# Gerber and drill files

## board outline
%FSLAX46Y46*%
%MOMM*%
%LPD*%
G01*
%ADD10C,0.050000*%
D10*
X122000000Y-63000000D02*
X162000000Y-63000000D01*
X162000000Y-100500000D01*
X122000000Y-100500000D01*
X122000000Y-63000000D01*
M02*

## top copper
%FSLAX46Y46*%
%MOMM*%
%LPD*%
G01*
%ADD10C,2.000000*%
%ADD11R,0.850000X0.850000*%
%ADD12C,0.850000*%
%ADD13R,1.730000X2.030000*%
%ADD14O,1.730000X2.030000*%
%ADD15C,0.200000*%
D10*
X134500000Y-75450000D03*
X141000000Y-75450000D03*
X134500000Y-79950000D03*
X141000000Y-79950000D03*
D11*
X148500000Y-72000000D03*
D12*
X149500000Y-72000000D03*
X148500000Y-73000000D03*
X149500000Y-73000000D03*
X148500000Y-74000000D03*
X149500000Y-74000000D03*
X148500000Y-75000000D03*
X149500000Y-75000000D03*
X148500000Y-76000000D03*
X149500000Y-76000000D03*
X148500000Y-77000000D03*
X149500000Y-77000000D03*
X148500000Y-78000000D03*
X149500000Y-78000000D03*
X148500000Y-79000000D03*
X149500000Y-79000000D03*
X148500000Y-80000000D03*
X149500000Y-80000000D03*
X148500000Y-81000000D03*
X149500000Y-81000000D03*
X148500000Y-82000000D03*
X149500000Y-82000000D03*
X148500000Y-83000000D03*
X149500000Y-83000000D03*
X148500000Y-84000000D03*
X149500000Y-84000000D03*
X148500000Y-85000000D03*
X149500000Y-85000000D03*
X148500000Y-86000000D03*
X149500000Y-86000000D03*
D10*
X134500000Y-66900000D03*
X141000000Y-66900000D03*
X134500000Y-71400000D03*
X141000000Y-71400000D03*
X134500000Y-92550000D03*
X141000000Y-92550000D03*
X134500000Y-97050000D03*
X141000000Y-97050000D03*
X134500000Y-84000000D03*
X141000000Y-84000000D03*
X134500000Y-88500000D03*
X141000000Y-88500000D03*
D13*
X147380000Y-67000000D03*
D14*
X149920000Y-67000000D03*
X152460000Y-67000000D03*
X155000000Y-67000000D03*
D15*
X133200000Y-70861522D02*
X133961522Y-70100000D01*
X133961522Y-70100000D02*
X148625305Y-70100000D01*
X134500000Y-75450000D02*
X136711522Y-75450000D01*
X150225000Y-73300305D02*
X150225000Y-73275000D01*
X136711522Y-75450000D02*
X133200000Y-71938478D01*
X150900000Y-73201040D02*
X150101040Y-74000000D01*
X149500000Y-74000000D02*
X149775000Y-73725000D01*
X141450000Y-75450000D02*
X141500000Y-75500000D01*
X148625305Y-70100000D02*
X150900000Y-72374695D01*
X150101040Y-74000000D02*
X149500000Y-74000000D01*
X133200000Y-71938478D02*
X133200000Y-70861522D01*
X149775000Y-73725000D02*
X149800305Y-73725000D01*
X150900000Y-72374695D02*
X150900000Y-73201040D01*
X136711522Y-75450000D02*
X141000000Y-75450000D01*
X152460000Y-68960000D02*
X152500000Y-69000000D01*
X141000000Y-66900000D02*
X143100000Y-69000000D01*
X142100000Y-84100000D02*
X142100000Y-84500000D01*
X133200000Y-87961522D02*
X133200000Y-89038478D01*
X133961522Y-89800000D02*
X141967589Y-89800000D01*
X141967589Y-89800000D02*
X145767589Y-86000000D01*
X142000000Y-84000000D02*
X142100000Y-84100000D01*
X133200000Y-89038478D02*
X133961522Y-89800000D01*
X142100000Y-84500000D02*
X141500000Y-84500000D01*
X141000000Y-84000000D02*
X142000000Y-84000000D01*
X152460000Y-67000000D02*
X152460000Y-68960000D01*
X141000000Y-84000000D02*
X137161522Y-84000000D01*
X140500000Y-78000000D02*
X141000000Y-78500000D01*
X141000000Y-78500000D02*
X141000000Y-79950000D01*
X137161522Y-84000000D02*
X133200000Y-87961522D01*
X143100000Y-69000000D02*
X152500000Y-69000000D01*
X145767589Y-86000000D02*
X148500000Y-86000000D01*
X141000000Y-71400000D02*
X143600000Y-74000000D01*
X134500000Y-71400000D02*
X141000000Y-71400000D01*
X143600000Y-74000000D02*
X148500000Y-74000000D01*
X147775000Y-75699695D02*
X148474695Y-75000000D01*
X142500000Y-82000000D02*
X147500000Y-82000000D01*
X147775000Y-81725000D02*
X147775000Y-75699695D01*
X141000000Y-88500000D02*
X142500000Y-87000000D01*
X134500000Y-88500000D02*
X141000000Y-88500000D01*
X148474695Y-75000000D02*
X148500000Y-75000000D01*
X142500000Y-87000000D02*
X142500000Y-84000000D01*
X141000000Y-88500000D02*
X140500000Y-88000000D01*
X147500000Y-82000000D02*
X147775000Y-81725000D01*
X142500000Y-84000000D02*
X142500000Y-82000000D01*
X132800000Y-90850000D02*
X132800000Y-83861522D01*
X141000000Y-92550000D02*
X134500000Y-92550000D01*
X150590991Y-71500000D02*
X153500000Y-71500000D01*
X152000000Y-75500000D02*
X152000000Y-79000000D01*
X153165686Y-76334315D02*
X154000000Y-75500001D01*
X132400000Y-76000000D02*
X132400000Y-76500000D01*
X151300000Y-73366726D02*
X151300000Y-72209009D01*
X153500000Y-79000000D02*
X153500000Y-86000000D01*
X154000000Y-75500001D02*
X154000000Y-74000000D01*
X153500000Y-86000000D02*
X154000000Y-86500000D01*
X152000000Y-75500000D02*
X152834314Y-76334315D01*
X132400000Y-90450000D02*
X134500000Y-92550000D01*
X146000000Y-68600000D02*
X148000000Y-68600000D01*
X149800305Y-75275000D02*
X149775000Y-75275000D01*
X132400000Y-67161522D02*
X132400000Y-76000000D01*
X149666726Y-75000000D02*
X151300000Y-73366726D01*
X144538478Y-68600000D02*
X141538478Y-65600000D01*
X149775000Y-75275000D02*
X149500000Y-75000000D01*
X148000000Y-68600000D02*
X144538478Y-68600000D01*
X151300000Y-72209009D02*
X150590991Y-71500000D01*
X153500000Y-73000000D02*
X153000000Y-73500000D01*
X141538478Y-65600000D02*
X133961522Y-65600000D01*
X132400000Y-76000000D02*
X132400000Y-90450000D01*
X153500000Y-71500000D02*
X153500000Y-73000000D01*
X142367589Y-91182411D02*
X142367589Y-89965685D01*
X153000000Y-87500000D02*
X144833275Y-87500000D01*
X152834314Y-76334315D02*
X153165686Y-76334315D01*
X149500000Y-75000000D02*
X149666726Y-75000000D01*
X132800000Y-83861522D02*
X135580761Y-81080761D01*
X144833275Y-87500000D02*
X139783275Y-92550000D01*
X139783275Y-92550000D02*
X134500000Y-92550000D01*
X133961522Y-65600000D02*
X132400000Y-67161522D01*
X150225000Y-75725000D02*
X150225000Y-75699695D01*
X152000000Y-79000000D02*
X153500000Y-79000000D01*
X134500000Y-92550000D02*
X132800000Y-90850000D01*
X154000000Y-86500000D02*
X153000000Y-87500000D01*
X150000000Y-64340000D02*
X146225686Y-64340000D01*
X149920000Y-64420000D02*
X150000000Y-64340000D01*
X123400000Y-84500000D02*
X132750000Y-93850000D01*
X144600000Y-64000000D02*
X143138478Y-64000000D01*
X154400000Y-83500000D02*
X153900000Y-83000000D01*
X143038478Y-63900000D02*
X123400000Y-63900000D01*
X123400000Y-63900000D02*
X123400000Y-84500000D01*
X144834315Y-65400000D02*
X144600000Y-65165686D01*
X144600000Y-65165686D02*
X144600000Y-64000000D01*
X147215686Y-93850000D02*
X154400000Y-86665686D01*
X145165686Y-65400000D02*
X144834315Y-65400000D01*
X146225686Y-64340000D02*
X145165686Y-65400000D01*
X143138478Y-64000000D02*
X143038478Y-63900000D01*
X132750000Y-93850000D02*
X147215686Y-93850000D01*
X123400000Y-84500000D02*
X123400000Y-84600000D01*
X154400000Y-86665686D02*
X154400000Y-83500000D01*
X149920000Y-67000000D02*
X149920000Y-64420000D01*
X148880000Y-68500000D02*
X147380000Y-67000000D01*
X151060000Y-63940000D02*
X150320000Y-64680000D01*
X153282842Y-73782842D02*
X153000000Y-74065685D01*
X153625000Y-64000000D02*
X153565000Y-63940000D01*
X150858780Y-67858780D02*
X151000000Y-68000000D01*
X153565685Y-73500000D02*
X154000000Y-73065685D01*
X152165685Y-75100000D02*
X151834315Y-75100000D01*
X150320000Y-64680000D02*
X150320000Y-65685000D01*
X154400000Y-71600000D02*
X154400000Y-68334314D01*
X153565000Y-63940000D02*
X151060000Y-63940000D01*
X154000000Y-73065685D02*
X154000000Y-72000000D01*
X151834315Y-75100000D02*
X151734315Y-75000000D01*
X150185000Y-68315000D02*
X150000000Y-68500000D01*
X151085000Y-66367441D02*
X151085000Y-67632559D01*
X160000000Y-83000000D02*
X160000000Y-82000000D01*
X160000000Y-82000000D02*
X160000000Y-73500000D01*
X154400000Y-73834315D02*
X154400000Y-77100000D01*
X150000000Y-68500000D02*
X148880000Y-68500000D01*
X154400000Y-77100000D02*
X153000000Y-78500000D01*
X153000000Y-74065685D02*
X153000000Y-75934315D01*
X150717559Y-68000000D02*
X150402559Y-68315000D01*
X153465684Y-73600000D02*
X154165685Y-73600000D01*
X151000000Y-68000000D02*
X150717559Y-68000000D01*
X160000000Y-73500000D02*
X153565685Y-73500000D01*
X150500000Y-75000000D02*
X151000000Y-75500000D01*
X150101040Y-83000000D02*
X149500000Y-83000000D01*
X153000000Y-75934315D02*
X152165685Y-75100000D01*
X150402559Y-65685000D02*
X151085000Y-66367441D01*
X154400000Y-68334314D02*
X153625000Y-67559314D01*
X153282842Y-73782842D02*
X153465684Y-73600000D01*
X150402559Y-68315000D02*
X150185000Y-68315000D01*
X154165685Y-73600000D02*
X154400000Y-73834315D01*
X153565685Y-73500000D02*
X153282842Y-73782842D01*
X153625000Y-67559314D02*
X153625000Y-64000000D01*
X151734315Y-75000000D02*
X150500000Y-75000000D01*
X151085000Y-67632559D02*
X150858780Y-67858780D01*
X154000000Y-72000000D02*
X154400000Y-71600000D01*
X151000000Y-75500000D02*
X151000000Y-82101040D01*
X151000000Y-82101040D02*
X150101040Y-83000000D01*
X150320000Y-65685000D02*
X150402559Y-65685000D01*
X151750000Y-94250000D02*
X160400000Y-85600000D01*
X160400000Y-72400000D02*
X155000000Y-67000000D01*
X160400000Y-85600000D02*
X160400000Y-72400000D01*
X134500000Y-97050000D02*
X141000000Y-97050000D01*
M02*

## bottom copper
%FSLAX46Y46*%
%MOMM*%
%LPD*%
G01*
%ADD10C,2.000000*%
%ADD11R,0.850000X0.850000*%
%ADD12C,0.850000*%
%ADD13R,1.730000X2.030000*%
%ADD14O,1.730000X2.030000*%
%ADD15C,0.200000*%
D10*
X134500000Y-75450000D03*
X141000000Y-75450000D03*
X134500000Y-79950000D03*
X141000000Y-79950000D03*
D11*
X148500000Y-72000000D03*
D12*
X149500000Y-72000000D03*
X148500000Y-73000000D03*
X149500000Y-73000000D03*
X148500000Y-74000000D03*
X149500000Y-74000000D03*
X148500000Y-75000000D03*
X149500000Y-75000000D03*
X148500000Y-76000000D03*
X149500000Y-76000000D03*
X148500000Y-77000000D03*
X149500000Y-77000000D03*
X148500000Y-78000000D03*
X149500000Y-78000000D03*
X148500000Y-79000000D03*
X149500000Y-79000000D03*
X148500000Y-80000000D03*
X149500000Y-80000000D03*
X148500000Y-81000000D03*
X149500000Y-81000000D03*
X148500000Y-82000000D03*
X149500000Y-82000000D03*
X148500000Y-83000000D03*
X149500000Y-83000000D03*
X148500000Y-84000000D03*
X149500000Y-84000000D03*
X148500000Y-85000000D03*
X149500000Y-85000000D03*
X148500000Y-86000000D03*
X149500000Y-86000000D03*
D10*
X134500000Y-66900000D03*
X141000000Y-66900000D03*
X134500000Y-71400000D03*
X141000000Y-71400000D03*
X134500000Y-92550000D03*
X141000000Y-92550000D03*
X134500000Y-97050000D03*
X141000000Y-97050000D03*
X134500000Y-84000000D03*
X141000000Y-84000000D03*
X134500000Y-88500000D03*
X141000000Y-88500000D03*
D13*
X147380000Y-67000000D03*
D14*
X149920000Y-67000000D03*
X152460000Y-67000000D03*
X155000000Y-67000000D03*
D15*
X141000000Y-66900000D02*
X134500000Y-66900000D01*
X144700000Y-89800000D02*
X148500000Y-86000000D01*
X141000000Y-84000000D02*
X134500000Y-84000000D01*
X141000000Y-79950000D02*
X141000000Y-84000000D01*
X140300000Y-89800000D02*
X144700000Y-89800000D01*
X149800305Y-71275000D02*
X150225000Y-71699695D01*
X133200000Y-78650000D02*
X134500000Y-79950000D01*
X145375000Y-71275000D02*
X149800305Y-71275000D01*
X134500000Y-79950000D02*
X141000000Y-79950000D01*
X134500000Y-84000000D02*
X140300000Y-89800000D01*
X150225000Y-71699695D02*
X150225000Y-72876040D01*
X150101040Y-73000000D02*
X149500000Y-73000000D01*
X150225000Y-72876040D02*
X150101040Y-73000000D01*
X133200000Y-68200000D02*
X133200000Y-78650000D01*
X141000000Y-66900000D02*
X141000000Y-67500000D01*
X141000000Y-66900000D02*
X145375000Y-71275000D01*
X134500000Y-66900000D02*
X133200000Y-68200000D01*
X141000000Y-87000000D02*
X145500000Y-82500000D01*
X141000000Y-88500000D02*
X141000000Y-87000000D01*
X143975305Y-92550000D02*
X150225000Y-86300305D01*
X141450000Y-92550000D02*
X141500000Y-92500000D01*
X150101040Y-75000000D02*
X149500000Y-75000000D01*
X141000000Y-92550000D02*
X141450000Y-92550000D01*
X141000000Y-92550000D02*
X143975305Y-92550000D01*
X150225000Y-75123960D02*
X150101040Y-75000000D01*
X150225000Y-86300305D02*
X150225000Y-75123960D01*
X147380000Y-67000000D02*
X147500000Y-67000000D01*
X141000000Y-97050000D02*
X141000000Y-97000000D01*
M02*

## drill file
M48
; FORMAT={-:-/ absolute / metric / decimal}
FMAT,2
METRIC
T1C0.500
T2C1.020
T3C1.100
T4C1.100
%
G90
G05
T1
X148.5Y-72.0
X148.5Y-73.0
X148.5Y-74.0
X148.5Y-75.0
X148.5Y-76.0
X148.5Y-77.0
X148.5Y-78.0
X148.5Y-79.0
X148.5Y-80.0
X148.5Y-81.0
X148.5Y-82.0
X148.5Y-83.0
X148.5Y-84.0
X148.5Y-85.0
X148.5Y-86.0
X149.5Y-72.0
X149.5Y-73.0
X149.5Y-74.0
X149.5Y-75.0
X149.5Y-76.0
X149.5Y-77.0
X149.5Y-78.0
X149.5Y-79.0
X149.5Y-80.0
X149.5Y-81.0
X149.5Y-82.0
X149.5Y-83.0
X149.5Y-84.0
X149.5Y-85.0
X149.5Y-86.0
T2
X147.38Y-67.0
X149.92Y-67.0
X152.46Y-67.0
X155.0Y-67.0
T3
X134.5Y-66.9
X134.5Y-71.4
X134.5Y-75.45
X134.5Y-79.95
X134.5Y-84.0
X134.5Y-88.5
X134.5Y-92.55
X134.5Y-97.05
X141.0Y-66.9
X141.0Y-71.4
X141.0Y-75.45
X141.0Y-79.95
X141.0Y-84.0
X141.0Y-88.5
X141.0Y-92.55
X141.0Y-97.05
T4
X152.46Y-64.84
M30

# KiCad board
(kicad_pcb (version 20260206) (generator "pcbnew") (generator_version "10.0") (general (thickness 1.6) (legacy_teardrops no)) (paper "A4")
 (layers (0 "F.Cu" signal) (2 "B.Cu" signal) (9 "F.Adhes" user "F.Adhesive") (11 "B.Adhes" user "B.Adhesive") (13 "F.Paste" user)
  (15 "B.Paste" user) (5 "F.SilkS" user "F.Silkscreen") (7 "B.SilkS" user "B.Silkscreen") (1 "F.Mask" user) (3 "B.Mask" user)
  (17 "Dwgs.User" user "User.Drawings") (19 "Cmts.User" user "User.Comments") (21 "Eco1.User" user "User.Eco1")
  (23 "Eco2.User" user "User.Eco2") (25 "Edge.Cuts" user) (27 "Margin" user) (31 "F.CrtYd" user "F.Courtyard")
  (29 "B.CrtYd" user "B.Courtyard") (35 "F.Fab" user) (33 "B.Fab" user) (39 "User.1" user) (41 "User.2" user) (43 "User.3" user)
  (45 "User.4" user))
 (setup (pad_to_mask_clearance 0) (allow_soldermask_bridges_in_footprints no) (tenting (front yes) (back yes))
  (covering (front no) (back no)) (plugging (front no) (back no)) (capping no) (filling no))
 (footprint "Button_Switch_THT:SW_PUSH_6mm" (layer "F.Cu") (at 134.5 75.45)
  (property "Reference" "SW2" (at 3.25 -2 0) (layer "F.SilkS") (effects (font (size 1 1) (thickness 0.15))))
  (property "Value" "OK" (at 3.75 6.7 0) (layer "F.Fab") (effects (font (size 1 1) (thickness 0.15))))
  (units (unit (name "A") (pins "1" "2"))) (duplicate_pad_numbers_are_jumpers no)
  (pad "1" thru_hole circle (at 0 0 90) (size 2 2) (drill 1.1) (layers "*.Cu" "*.Mask") (remove_unused_layers no) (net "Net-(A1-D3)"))
  (pad "1" thru_hole circle (at 6.5 0 90) (size 2 2) (drill 1.1) (layers "*.Cu" "*.Mask") (remove_unused_layers no) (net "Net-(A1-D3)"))
  (pad "2" thru_hole circle (at 0 4.5 90) (size 2 2) (drill 1.1) (layers "*.Cu" "*.Mask") (remove_unused_layers no) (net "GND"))
  (pad "2" thru_hole circle (at 6.5 4.5 90) (size 2 2) (drill 1.1) (layers "*.Cu" "*.Mask") (remove_unused_layers no) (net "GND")))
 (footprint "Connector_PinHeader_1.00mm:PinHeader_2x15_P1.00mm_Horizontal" (layer "F.Cu") (at 148.5 72)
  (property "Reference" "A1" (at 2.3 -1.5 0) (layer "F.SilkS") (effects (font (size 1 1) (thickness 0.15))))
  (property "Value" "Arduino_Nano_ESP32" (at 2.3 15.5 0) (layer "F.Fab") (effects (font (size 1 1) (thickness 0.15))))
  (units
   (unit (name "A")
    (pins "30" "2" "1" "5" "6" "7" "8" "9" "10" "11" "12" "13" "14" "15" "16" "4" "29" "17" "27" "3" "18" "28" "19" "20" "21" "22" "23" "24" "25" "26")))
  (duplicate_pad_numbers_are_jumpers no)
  (pad "1" thru_hole rect (at 0 0) (size 0.85 0.85) (drill 0.5) (layers "*.Cu" "*.Mask") (remove_unused_layers no)
   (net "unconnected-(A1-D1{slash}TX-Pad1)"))
  (pad "2" thru_hole circle (at 1 0) (size 0.85 0.85) (drill 0.5) (layers "*.Cu" "*.Mask") (remove_unused_layers no)
   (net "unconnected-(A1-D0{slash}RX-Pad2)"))
  (pad "3" thru_hole circle (at 0 1) (size 0.85 0.85) (drill 0.5) (layers "*.Cu" "*.Mask") (remove_unused_layers no)
   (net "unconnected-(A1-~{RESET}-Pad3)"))
  (pad "4" thru_hole circle (at 1 1) (size 0.85 0.85) (drill 0.5) (layers "*.Cu" "*.Mask") (remove_unused_layers no) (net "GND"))
  (pad "5" thru_hole circle (at 0 2) (size 0.85 0.85) (drill 0.5) (layers "*.Cu" "*.Mask") (remove_unused_layers no) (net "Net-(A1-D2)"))
  (pad "6" thru_hole circle (at 1 2) (size 0.85 0.85) (drill 0.5) (layers "*.Cu" "*.Mask") (remove_unused_layers no) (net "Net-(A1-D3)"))
  (pad "7" thru_hole circle (at 0 3) (size 0.85 0.85) (drill 0.5) (layers "*.Cu" "*.Mask") (remove_unused_layers no) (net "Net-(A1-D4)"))
  (pad "8" thru_hole circle (at 1 3) (size 0.85 0.85) (drill 0.5) (layers "*.Cu" "*.Mask") (remove_unused_layers no) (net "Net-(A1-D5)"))
  (pad "9" thru_hole circle (at 0 4) (size 0.85 0.85) (drill 0.5) (layers "*.Cu" "*.Mask") (remove_unused_layers no)
   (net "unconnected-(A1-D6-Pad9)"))
  (pad "10" thru_hole circle (at 1 4) (size 0.85 0.85) (drill 0.5) (layers "*.Cu" "*.Mask") (remove_unused_layers no)
   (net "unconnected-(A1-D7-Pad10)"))
  (pad "11" thru_hole circle (at 0 5) (size 0.85 0.85) (drill 0.5) (layers "*.Cu" "*.Mask") (remove_unused_layers no)
   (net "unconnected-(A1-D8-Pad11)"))
  (pad "12" thru_hole circle (at 1 5) (size 0.85 0.85) (drill 0.5) (layers "*.Cu" "*.Mask") (remove_unused_layers no)
   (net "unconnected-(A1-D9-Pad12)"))
  (pad "13" thru_hole circle (at 0 6) (size 0.85 0.85) (drill 0.5) (layers "*.Cu" "*.Mask") (remove_unused_layers no)
   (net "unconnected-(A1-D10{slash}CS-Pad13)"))
  (pad "14" thru_hole circle (at 1 6) (size 0.85 0.85) (drill 0.5) (layers "*.Cu" "*.Mask") (remove_unused_layers no)
   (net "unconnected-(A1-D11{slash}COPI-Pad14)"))
  (pad "15" thru_hole circle (at 0 7) (size 0.85 0.85) (drill 0.5) (layers "*.Cu" "*.Mask") (remove_unused_layers no)
   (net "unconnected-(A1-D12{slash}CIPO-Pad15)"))
  (pad "16" thru_hole circle (at 1 7) (size 0.85 0.85) (drill 0.5) (layers "*.Cu" "*.Mask") (remove_unused_layers no)
   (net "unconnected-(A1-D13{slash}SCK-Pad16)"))
  (pad "17" thru_hole circle (at 0 8) (size 0.85 0.85) (drill 0.5) (layers "*.Cu" "*.Mask") (remove_unused_layers no)
   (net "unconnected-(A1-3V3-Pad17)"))
  (pad "18" thru_hole circle (at 1 8) (size 0.85 0.85) (drill 0.5) (layers "*.Cu" "*.Mask") (remove_unused_layers no)
   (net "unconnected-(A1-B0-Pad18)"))
  (pad "19" thru_hole circle (at 0 9) (size 0.85 0.85) (drill 0.5) (layers "*.Cu" "*.Mask") (remove_unused_layers no)
   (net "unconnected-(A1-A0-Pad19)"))
  (pad "20" thru_hole circle (at 1 9) (size 0.85 0.85) (drill 0.5) (layers "*.Cu" "*.Mask") (remove_unused_layers no)
   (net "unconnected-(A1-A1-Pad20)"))
  (pad "21" thru_hole circle (at 0 10) (size 0.85 0.85) (drill 0.5) (layers "*.Cu" "*.Mask") (remove_unused_layers no)
   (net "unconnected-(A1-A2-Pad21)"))
  (pad "22" thru_hole circle (at 1 10) (size 0.85 0.85) (drill 0.5) (layers "*.Cu" "*.Mask") (remove_unused_layers no)
   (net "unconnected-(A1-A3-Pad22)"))
  (pad "23" thru_hole circle (at 0 11) (size 0.85 0.85) (drill 0.5) (layers "*.Cu" "*.Mask") (remove_unused_layers no)
   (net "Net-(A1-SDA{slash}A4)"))
  (pad "24" thru_hole circle (at 1 11) (size 0.85 0.85) (drill 0.5) (layers "*.Cu" "*.Mask") (remove_unused_layers no)
   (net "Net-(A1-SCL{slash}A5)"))
  (pad "25" thru_hole circle (at 0 12) (size 0.85 0.85) (drill 0.5) (layers "*.Cu" "*.Mask") (remove_unused_layers no)
   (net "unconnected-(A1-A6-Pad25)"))
  (pad "26" thru_hole circle (at 1 12) (size 0.85 0.85) (drill 0.5) (layers "*.Cu" "*.Mask") (remove_unused_layers no)
   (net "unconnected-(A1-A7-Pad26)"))
  (pad "27" thru_hole circle (at 0 13) (size 0.85 0.85) (drill 0.5) (layers "*.Cu" "*.Mask") (remove_unused_layers no)
   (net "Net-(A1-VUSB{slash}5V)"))
  (pad "28" thru_hole circle (at 1 13) (size 0.85 0.85) (drill 0.5) (layers "*.Cu" "*.Mask") (remove_unused_layers no)
   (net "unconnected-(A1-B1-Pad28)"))
  (pad "29" thru_hole circle (at 0 14) (size 0.85 0.85) (drill 0.5) (layers "*.Cu" "*.Mask") (remove_unused_layers no) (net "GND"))
  (pad "30" thru_hole circle (at 1 14) (size 0.85 0.85) (drill 0.5) (layers "*.Cu" "*.Mask") (remove_unused_layers no)
   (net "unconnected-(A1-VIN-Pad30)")))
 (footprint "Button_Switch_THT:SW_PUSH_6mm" (layer "F.Cu") (at 134.5 66.9)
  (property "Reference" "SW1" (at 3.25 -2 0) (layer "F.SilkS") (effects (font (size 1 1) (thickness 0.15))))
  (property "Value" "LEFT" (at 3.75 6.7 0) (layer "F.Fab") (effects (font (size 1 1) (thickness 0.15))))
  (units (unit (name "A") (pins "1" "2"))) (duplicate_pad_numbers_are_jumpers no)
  (pad "1" thru_hole circle (at 0 0 90) (size 2 2) (drill 1.1) (layers "*.Cu" "*.Mask") (remove_unused_layers no) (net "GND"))
  (pad "1" thru_hole circle (at 6.5 0 90) (size 2 2) (drill 1.1) (layers "*.Cu" "*.Mask") (remove_unused_layers no) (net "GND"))
  (pad "2" thru_hole circle (at 0 4.5 90) (size 2 2) (drill 1.1) (layers "*.Cu" "*.Mask") (remove_unused_layers no) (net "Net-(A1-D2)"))
  (pad "2" thru_hole circle (at 6.5 4.5 90) (size 2 2) (drill 1.1) (layers "*.Cu" "*.Mask") (remove_unused_layers no) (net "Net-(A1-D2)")))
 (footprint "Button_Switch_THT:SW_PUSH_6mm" (layer "F.Cu") (at 134.5 92.55)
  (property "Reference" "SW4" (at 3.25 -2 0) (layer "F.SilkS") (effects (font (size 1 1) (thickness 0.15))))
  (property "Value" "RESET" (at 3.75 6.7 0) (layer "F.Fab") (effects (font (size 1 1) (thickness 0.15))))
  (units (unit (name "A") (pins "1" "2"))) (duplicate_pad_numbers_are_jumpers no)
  (pad "1" thru_hole circle (at 0 0 90) (size 2 2) (drill 1.1) (layers "*.Cu" "*.Mask") (remove_unused_layers no) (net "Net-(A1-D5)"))
  (pad "1" thru_hole circle (at 6.5 0 90) (size 2 2) (drill 1.1) (layers "*.Cu" "*.Mask") (remove_unused_layers no) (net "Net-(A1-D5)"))
  (pad "2" thru_hole circle (at 0 4.5 90) (size 2 2) (drill 1.1) (layers "*.Cu" "*.Mask") (remove_unused_layers no)
   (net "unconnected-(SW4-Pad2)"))
  (pad "2" thru_hole circle (at 6.5 4.5 90) (size 2 2) (drill 1.1) (layers "*.Cu" "*.Mask") (remove_unused_layers no)
   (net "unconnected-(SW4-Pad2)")))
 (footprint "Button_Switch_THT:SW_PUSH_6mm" (layer "F.Cu") (at 134.5 84)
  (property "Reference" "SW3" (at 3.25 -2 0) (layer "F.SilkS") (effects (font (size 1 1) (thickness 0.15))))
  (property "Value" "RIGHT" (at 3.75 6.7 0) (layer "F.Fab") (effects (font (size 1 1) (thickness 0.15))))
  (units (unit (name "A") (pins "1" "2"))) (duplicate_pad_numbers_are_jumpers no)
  (pad "1" thru_hole circle (at 0 0 90) (size 2 2) (drill 1.1) (layers "*.Cu" "*.Mask") (remove_unused_layers no) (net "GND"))
  (pad "1" thru_hole circle (at 6.5 0 90) (size 2 2) (drill 1.1) (layers "*.Cu" "*.Mask") (remove_unused_layers no) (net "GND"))
  (pad "2" thru_hole circle (at 0 4.5 90) (size 2 2) (drill 1.1) (layers "*.Cu" "*.Mask") (remove_unused_layers no) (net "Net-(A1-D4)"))
  (pad "2" thru_hole circle (at 6.5 4.5 90) (size 2 2) (drill 1.1) (layers "*.Cu" "*.Mask") (remove_unused_layers no) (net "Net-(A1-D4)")))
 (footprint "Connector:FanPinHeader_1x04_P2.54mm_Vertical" (layer "F.Cu") (at 147.38 67)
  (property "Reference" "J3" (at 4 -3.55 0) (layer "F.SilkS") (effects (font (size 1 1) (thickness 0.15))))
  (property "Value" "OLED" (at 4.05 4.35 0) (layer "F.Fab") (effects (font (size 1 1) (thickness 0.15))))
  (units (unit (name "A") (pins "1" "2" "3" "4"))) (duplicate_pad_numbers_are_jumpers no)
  (pad "" np_thru_hole circle (at 5.08 -2.16 90) (size 1.1 1.1) (drill 1.1) (layers "*.Cu" "*.Mask"))
  (pad "1" thru_hole rect (at 0 0 90) (size 2.03 1.73) (drill 1.02) (layers "*.Cu" "*.Mask") (remove_unused_layers no)
   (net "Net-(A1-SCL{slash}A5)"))
  (pad "2" thru_hole oval (at 2.54 0 90) (size 2.03 1.73) (drill 1.02) (layers "*.Cu" "*.Mask") (remove_unused_layers no)
   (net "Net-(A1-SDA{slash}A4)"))
  (pad "3" thru_hole oval (at 5.08 0 90) (size 2.03 1.73) (drill 1.02) (layers "*.Cu" "*.Mask") (remove_unused_layers no) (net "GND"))
  (pad "4" thru_hole oval (at 7.62 0 90) (size 2.03 1.73) (drill 1.02) (layers "*.Cu" "*.Mask") (remove_unused_layers no)
   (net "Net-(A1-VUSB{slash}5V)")))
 (gr_rect (start 122 63) (end 162 100.5) (stroke (width 0.05) (type default)) (fill no) (layer "Edge.Cuts"))
 (segment (start 133.2 70.861522) (end 133.961522 70.1) (width 0.2) (layer "F.Cu") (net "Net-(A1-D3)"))
 (segment (start 133.961522 70.1) (end 148.625305 70.1) (width 0.2) (layer "F.Cu") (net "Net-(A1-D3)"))
 (segment (start 134.5 75.45) (end 136.711522 75.45) (width 0.2) (layer "F.Cu") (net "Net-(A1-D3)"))
 (segment (start 150.225 73.300305) (end 150.225 73.275) (width 0.2) (layer "F.Cu") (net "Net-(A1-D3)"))
 (segment (start 136.711522 75.45) (end 133.2 71.938478) (width 0.2) (layer "F.Cu") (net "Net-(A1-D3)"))
 (segment (start 150.9 73.20104) (end 150.10104 74) (width 0.2) (layer "F.Cu") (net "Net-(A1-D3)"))
 (segment (start 149.5 74) (end 149.775 73.725) (width 0.2) (layer "F.Cu") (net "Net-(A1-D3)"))
 (segment (start 141.45 75.45) (end 141.5 75.5) (width 0.2) (layer "F.Cu") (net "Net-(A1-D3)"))
 (segment (start 148.625305 70.1) (end 150.9 72.374695) (width 0.2) (layer "F.Cu") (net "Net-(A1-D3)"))
 (segment (start 150.10104 74) (end 149.5 74) (width 0.2) (layer "F.Cu") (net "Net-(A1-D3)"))
 (segment (start 133.2 71.938478) (end 133.2 70.861522) (width 0.2) (layer "F.Cu") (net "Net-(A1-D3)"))
 (segment (start 149.775 73.725) (end 149.800305 73.725) (width 0.2) (layer "F.Cu") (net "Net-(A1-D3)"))
 (segment (start 150.9 72.374695) (end 150.9 73.20104) (width 0.2) (layer "F.Cu") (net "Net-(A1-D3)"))
 (segment (start 136.711522 75.45) (end 141 75.45) (width 0.2) (layer "F.Cu") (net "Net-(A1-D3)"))
 (segment (start 152.46 68.96) (end 152.5 69) (width 0.2) (layer "F.Cu") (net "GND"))
 (segment (start 141 66.9) (end 143.1 69) (width 0.2) (layer "F.Cu") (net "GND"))
 (segment (start 142.1 84.1) (end 142.1 84.5) (width 0.2) (layer "F.Cu") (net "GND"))
 (segment (start 133.2 87.961522) (end 133.2 89.038478) (width 0.2) (layer "F.Cu") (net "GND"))
 (segment (start 133.961522 89.8) (end 141.967589 89.8) (width 0.2) (layer "F.Cu") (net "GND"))
 (segment (start 141.967589 89.8) (end 145.767589 86) (width 0.2) (layer "F.Cu") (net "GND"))
 (segment (start 142 84) (end 142.1 84.1) (width 0.2) (layer "F.Cu") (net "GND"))
 (segment (start 133.2 89.038478) (end 133.961522 89.8) (width 0.2) (layer "F.Cu") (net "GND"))
 (segment (start 142.1 84.5) (end 141.5 84.5) (width 0.2) (layer "F.Cu") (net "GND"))
 (segment (start 141 84) (end 142 84) (width 0.2) (layer "F.Cu") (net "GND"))
 (segment (start 152.46 67) (end 152.46 68.96) (width 0.2) (layer "F.Cu") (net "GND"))
 (segment (start 141 84) (end 137.161522 84) (width 0.2) (layer "F.Cu") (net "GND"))
 (segment (start 140.5 78) (end 141 78.5) (width 0.2) (layer "F.Cu") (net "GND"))
 (segment (start 141 78.5) (end 141 79.95) (width 0.2) (layer "F.Cu") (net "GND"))
 (segment (start 137.161522 84) (end 133.2 87.961522) (width 0.2) (layer "F.Cu") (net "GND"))
 (segment (start 143.1 69) (end 152.5 69) (width 0.2) (layer "F.Cu") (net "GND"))
 (segment (start 145.767589 86) (end 148.5 86) (width 0.2) (layer "F.Cu") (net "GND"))
 (segment (start 141 66.9) (end 134.5 66.9) (width 0.2) (layer "B.Cu") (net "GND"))
 (segment (start 144.7 89.8) (end 148.5 86) (width 0.2) (layer "B.Cu") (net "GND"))
 (segment (start 141 84) (end 134.5 84) (width 0.2) (layer "B.Cu") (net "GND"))
 (segment (start 141 79.95) (end 141 84) (width 0.2) (layer "B.Cu") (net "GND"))
 (segment (start 140.3 89.8) (end 144.7 89.8) (width 0.2) (layer "B.Cu") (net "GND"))
 (segment (start 149.800305 71.275) (end 150.225 71.699695) (width 0.2) (layer "B.Cu") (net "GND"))
 (segment (start 133.2 78.65) (end 134.5 79.95) (width 0.2) (layer "B.Cu") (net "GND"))
 (segment (start 145.375 71.275) (end 149.800305 71.275) (width 0.2) (layer "B.Cu") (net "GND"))
 (segment (start 134.5 79.95) (end 141 79.95) (width 0.2) (layer "B.Cu") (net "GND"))
 (segment (start 134.5 84) (end 140.3 89.8) (width 0.2) (layer "B.Cu") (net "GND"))
 (segment (start 150.225 71.699695) (end 150.225 72.87604) (width 0.2) (layer "B.Cu") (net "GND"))
 (segment (start 150.10104 73) (end 149.5 73) (width 0.2) (layer "B.Cu") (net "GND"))
 (segment (start 150.225 72.87604) (end 150.10104 73) (width 0.2) (layer "B.Cu") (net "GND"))
 (segment (start 133.2 68.2) (end 133.2 78.65) (width 0.2) (layer "B.Cu") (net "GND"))
 (segment (start 141 66.9) (end 141 67.5) (width 0.2) (layer "B.Cu") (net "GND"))
 (segment (start 141 66.9) (end 145.375 71.275) (width 0.2) (layer "B.Cu") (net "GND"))
 (segment (start 134.5 66.9) (end 133.2 68.2) (width 0.2) (layer "B.Cu") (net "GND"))
 (segment (start 141 71.4) (end 143.6 74) (width 0.2) (layer "F.Cu") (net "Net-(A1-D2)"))
 (segment (start 134.5 71.4) (end 141 71.4) (width 0.2) (layer "F.Cu") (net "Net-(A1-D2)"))
 (segment (start 143.6 74) (end 148.5 74) (width 0.2) (layer "F.Cu") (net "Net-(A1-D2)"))
 (segment (start 147.775 75.699695) (end 148.474695 75) (width 0.2) (layer "F.Cu") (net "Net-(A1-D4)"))
 (segment (start 142.5 82) (end 147.5 82) (width 0.2) (layer "F.Cu") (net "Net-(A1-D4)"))
 (segment (start 147.775 81.725) (end 147.775 75.699695) (width 0.2) (layer "F.Cu") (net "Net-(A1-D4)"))
 (segment (start 141 88.5) (end 142.5 87) (width 0.2) (layer "F.Cu") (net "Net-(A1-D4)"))
 (segment (start 134.5 88.5) (end 141 88.5) (width 0.2) (layer "F.Cu") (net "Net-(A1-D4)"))
 (segment (start 148.474695 75) (end 148.5 75) (width 0.2) (layer "F.Cu") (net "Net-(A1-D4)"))
 (segment (start 142.5 87) (end 142.5 84) (width 0.2) (layer "F.Cu") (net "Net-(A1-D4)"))
 (segment (start 141 88.5) (end 140.5 88) (width 0.2) (layer "F.Cu") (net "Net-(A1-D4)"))
 (segment (start 147.5 82) (end 147.775 81.725) (width 0.2) (layer "F.Cu") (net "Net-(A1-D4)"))
 (segment (start 142.5 84) (end 142.5 82) (width 0.2) (layer "F.Cu") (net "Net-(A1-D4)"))
 (segment (start 141 87) (end 145.5 82.5) (width 0.2) (layer "B.Cu") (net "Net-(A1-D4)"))
 (segment (start 141 88.5) (end 141 87) (width 0.2) (layer "B.Cu") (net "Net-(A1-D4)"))
 (segment (start 132.8 90.85) (end 132.8 83.861522) (width 0.2) (layer "F.Cu") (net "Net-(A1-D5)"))
 (segment (start 141 92.55) (end 134.5 92.55) (width 0.2) (layer "F.Cu") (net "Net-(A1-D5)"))
 (segment (start 150.590991 71.5) (end 153.5 71.5) (width 0.2) (layer "F.Cu") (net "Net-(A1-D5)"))
 (segment (start 152 75.5) (end 152 79) (width 0.2) (layer "F.Cu") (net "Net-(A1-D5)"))
 (segment (start 153.165686 76.334315) (end 154 75.500001) (width 0.2) (layer "F.Cu") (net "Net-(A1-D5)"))
 (segment (start 132.4 76) (end 132.4 76.5) (width 0.2) (layer "F.Cu") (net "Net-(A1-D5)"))
 (segment (start 151.3 73.366726) (end 151.3 72.209009) (width 0.2) (layer "F.Cu") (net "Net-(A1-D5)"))
 (segment (start 153.5 79) (end 153.5 86) (width 0.2) (layer "F.Cu") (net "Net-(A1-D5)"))
 (segment (start 154 75.500001) (end 154 74) (width 0.2) (layer "F.Cu") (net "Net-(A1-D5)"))
 (segment (start 153.5 86) (end 154 86.5) (width 0.2) (layer "F.Cu") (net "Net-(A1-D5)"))
 (segment (start 152 75.5) (end 152.834314 76.334315) (width 0.2) (layer "F.Cu") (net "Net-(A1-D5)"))
 (segment (start 132.4 90.45) (end 134.5 92.55) (width 0.2) (layer "F.Cu") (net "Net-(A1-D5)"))
 (segment (start 146 68.6) (end 148 68.6) (width 0.2) (layer "F.Cu") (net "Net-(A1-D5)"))
 (segment (start 149.800305 75.275) (end 149.775 75.275) (width 0.2) (layer "F.Cu") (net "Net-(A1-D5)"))
 (segment (start 132.4 67.161522) (end 132.4 76) (width 0.2) (layer "F.Cu") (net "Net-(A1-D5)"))
 (segment (start 149.666726 75) (end 151.3 73.366726) (width 0.2) (layer "F.Cu") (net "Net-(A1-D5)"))
 (segment (start 144.538478 68.6) (end 141.538478 65.6) (width 0.2) (layer "F.Cu") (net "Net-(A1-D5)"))
 (segment (start 149.775 75.275) (end 149.5 75) (width 0.2) (layer "F.Cu") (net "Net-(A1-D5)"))
 (segment (start 148 68.6) (end 144.538478 68.6) (width 0.2) (layer "F.Cu") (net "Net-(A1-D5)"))
 (segment (start 151.3 72.209009) (end 150.590991 71.5) (width 0.2) (layer "F.Cu") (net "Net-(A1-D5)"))
 (segment (start 153.5 73) (end 153 73.5) (width 0.2) (layer "F.Cu") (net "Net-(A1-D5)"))
 (segment (start 141.538478 65.6) (end 133.961522 65.6) (width 0.2) (layer "F.Cu") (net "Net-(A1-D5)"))
 (segment (start 132.4 76) (end 132.4 90.45) (width 0.2) (layer "F.Cu") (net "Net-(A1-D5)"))
 (segment (start 153.5 71.5) (end 153.5 73) (width 0.2) (layer "F.Cu") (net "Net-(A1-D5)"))
 (segment (start 142.367589 91.182411) (end 142.367589 89.965685) (width 0.2) (layer "F.Cu") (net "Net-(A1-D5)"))
 (segment (start 153 87.5) (end 144.833275 87.5) (width 0.2) (layer "F.Cu") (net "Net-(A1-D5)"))
 (segment (start 152.834314 76.334315) (end 153.165686 76.334315) (width 0.2) (layer "F.Cu") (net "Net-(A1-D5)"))
 (segment (start 149.5 75) (end 149.666726 75) (width 0.2) (layer "F.Cu") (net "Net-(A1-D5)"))
 (segment (start 132.8 83.861522) (end 135.580761 81.080761) (width 0.2) (layer "F.Cu") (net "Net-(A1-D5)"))
 (segment (start 144.833275 87.5) (end 139.783275 92.55) (width 0.2) (layer "F.Cu") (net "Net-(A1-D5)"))
 (segment (start 139.783275 92.55) (end 134.5 92.55) (width 0.2) (layer "F.Cu") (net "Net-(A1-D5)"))
 (segment (start 133.961522 65.6) (end 132.4 67.161522) (width 0.2) (layer "F.Cu") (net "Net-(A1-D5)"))
 (segment (start 150.225 75.725) (end 150.225 75.699695) (width 0.2) (layer "F.Cu") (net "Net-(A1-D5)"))
 (segment (start 152 79) (end 153.5 79) (width 0.2) (layer "F.Cu") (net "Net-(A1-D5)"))
 (segment (start 134.5 92.55) (end 132.8 90.85) (width 0.2) (layer "F.Cu") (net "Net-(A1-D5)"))
 (segment (start 154 86.5) (end 153 87.5) (width 0.2) (layer "F.Cu") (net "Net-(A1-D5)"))
 (segment (start 143.975305 92.55) (end 150.225 86.300305) (width 0.2) (layer "B.Cu") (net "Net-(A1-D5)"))
 (segment (start 141.45 92.55) (end 141.5 92.5) (width 0.2) (layer "B.Cu") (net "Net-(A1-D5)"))
 (segment (start 150.10104 75) (end 149.5 75) (width 0.2) (layer "B.Cu") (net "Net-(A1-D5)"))
 (segment (start 141 92.55) (end 141.45 92.55) (width 0.2) (layer "B.Cu") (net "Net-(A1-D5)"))
 (segment (start 141 92.55) (end 143.975305 92.55) (width 0.2) (layer "B.Cu") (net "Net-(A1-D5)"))
 (segment (start 150.225 75.12396) (end 150.10104 75) (width 0.2) (layer "B.Cu") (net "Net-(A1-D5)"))
 (segment (start 150.225 86.300305) (end 150.225 75.12396) (width 0.2) (layer "B.Cu") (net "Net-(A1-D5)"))
 (segment (start 150 64.34) (end 146.225686 64.34) (width 0.2) (layer "F.Cu") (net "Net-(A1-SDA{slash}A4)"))
 (segment (start 149.92 64.42) (end 150 64.34) (width 0.2) (layer "F.Cu") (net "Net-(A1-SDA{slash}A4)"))
 (segment (start 123.4 84.5) (end 132.75 93.85) (width 0.2) (layer "F.Cu") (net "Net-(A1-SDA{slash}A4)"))
 (segment (start 144.6 64) (end 143.138478 64) (width 0.2) (layer "F.Cu") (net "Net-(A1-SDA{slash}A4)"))
 (segment (start 154.4 83.5) (end 153.9 83) (width 0.2) (layer "F.Cu") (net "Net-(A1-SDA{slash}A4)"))
 (segment (start 143.038478 63.9) (end 123.4 63.9) (width 0.2) (layer "F.Cu") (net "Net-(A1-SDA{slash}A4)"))
 (segment (start 123.4 63.9) (end 123.4 84.5) (width 0.2) (layer "F.Cu") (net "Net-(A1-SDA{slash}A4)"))
 (segment (start 144.834315 65.4) (end 144.6 65.165686) (width 0.2) (layer "F.Cu") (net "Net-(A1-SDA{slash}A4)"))
 (segment (start 144.6 65.165686) (end 144.6 64) (width 0.2) (layer "F.Cu") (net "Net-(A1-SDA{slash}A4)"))
 (segment (start 147.215686 93.85) (end 154.4 86.665686) (width 0.2) (layer "F.Cu") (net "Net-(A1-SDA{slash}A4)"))
 (segment (start 145.165686 65.4) (end 144.834315 65.4) (width 0.2) (layer "F.Cu") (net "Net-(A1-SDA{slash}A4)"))
 (segment (start 146.225686 64.34) (end 145.165686 65.4) (width 0.2) (layer "F.Cu") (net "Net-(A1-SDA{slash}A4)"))
 (segment (start 143.138478 64) (end 143.038478 63.9) (width 0.2) (layer "F.Cu") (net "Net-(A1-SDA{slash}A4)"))
 (segment (start 132.75 93.85) (end 147.215686 93.85) (width 0.2) (layer "F.Cu") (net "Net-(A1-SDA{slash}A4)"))
 (segment (start 123.4 84.5) (end 123.4 84.6) (width 0.2) (layer "F.Cu") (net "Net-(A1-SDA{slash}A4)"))
 (segment (start 154.4 86.665686) (end 154.4 83.5) (width 0.2) (layer "F.Cu") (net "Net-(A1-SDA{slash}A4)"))
 (segment (start 149.92 67) (end 149.92 64.42) (width 0.2) (layer "F.Cu") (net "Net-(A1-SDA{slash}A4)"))
 (segment (start 148.88 68.5) (end 147.38 67) (width 0.2) (layer "F.Cu") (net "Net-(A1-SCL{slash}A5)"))
 (segment (start 151.06 63.94) (end 150.32 64.68) (width 0.2) (layer "F.Cu") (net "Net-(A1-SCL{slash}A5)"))
 (segment (start 153.282842 73.782842) (end 153 74.065685) (width 0.2) (layer "F.Cu") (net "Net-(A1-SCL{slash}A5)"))
 (segment (start 153.625 64) (end 153.565 63.94) (width 0.2) (layer "F.Cu") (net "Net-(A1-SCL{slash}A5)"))
 (segment (start 150.85878 67.85878) (end 151 68) (width 0.2) (layer "F.Cu") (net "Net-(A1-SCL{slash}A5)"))
 (segment (start 153.565685 73.5) (end 154 73.065685) (width 0.2) (layer "F.Cu") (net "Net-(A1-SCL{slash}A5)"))
 (segment (start 152.165685 75.1) (end 151.834315 75.1) (width 0.2) (layer "F.Cu") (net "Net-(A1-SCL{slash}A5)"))
 (segment (start 150.32 64.68) (end 150.32 65.685) (width 0.2) (layer "F.Cu") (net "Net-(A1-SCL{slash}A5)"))
 (segment (start 154.4 71.6) (end 154.4 68.334314) (width 0.2) (layer "F.Cu") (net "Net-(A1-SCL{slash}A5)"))
 (segment (start 153.565 63.94) (end 151.06 63.94) (width 0.2) (layer "F.Cu") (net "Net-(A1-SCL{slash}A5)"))
 (segment (start 154 73.065685) (end 154 72) (width 0.2) (layer "F.Cu") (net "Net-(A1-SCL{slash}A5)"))
 (segment (start 151.834315 75.1) (end 151.734315 75) (width 0.2) (layer "F.Cu") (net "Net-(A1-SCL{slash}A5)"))
 (segment (start 150.185 68.315) (end 150 68.5) (width 0.2) (layer "F.Cu") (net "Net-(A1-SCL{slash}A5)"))
 (segment (start 151.085 66.367441) (end 151.085 67.632559) (width 0.2) (layer "F.Cu") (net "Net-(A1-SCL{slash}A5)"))
 (segment (start 160 83) (end 160 82) (width 0.2) (layer "F.Cu") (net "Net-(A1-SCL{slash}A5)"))
 (segment (start 160 82) (end 160 73.5) (width 0.2) (layer "F.Cu") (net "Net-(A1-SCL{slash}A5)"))
 (segment (start 154.4 73.834315) (end 154.4 77.1) (width 0.2) (layer "F.Cu") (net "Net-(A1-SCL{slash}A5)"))
 (segment (start 150 68.5) (end 148.88 68.5) (width 0.2) (layer "F.Cu") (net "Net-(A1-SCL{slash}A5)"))
 (segment (start 154.4 77.1) (end 153 78.5) (width 0.2) (layer "F.Cu") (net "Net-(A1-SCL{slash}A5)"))
 (segment (start 153 74.065685) (end 153 75.934315) (width 0.2) (layer "F.Cu") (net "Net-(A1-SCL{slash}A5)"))
 (segment (start 150.717559 68) (end 150.402559 68.315) (width 0.2) (layer "F.Cu") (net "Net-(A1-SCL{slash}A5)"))
 (segment (start 153.465684 73.6) (end 154.165685 73.6) (width 0.2) (layer "F.Cu") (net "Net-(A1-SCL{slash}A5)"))
 (segment (start 151 68) (end 150.717559 68) (width 0.2) (layer "F.Cu") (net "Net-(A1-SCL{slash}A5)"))
 (segment (start 160 73.5) (end 153.565685 73.5) (width 0.2) (layer "F.Cu") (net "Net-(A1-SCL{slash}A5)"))
 (segment (start 150.5 75) (end 151 75.5) (width 0.2) (layer "F.Cu") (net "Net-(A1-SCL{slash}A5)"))
 (segment (start 150.10104 83) (end 149.5 83) (width 0.2) (layer "F.Cu") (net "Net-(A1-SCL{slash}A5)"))
 (segment (start 153 75.934315) (end 152.165685 75.1) (width 0.2) (layer "F.Cu") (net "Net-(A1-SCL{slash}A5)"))
 (segment (start 150.402559 65.685) (end 151.085 66.367441) (width 0.2) (layer "F.Cu") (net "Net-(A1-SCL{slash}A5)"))
 (segment (start 154.4 68.334314) (end 153.625 67.559314) (width 0.2) (layer "F.Cu") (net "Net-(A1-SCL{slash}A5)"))
 (segment (start 153.282842 73.782842) (end 153.465684 73.6) (width 0.2) (layer "F.Cu") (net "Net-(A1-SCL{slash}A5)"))
 (segment (start 150.402559 68.315) (end 150.185 68.315) (width 0.2) (layer "F.Cu") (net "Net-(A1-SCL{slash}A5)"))
 (segment (start 154.165685 73.6) (end 154.4 73.834315) (width 0.2) (layer "F.Cu") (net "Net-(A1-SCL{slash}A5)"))
 (segment (start 153.565685 73.5) (end 153.282842 73.782842) (width 0.2) (layer "F.Cu") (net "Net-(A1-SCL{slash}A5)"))
 (segment (start 153.625 67.559314) (end 153.625 64) (width 0.2) (layer "F.Cu") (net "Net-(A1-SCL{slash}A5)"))
 (segment (start 151.734315 75) (end 150.5 75) (width 0.2) (layer "F.Cu") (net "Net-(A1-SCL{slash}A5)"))
 (segment (start 151.085 67.632559) (end 150.85878 67.85878) (width 0.2) (layer "F.Cu") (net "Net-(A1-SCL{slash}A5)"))
 (segment (start 154 72) (end 154.4 71.6) (width 0.2) (layer "F.Cu") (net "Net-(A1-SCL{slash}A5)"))
 (segment (start 151 75.5) (end 151 82.10104) (width 0.2) (layer "F.Cu") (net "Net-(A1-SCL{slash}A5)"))
 (segment (start 151 82.10104) (end 150.10104 83) (width 0.2) (layer "F.Cu") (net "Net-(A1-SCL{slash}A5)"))
 (segment (start 150.32 65.685) (end 150.402559 65.685) (width 0.2) (layer "F.Cu") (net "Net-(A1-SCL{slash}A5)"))
 (segment (start 147.38 67) (end 147.5 67) (width 0.2) (layer "B.Cu") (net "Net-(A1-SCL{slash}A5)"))
 (segment (start 151.75 94.25) (end 160.4 85.6) (width 0.2) (layer "F.Cu") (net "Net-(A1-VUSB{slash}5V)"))
 (segment (start 160.4 72.4) (end 155 67) (width 0.2) (layer "F.Cu") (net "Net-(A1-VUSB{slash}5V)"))
 (segment (start 160.4 85.6) (end 160.4 72.4) (width 0.2) (layer "F.Cu") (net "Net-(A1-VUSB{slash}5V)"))
 (segment (start 134.5 97.05) (end 141 97.05) (width 0.2) (layer "F.Cu") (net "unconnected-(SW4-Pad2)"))
 (segment (start 141 97.05) (end 141 97) (width 0.2) (layer "B.Cu") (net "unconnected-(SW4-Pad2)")))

